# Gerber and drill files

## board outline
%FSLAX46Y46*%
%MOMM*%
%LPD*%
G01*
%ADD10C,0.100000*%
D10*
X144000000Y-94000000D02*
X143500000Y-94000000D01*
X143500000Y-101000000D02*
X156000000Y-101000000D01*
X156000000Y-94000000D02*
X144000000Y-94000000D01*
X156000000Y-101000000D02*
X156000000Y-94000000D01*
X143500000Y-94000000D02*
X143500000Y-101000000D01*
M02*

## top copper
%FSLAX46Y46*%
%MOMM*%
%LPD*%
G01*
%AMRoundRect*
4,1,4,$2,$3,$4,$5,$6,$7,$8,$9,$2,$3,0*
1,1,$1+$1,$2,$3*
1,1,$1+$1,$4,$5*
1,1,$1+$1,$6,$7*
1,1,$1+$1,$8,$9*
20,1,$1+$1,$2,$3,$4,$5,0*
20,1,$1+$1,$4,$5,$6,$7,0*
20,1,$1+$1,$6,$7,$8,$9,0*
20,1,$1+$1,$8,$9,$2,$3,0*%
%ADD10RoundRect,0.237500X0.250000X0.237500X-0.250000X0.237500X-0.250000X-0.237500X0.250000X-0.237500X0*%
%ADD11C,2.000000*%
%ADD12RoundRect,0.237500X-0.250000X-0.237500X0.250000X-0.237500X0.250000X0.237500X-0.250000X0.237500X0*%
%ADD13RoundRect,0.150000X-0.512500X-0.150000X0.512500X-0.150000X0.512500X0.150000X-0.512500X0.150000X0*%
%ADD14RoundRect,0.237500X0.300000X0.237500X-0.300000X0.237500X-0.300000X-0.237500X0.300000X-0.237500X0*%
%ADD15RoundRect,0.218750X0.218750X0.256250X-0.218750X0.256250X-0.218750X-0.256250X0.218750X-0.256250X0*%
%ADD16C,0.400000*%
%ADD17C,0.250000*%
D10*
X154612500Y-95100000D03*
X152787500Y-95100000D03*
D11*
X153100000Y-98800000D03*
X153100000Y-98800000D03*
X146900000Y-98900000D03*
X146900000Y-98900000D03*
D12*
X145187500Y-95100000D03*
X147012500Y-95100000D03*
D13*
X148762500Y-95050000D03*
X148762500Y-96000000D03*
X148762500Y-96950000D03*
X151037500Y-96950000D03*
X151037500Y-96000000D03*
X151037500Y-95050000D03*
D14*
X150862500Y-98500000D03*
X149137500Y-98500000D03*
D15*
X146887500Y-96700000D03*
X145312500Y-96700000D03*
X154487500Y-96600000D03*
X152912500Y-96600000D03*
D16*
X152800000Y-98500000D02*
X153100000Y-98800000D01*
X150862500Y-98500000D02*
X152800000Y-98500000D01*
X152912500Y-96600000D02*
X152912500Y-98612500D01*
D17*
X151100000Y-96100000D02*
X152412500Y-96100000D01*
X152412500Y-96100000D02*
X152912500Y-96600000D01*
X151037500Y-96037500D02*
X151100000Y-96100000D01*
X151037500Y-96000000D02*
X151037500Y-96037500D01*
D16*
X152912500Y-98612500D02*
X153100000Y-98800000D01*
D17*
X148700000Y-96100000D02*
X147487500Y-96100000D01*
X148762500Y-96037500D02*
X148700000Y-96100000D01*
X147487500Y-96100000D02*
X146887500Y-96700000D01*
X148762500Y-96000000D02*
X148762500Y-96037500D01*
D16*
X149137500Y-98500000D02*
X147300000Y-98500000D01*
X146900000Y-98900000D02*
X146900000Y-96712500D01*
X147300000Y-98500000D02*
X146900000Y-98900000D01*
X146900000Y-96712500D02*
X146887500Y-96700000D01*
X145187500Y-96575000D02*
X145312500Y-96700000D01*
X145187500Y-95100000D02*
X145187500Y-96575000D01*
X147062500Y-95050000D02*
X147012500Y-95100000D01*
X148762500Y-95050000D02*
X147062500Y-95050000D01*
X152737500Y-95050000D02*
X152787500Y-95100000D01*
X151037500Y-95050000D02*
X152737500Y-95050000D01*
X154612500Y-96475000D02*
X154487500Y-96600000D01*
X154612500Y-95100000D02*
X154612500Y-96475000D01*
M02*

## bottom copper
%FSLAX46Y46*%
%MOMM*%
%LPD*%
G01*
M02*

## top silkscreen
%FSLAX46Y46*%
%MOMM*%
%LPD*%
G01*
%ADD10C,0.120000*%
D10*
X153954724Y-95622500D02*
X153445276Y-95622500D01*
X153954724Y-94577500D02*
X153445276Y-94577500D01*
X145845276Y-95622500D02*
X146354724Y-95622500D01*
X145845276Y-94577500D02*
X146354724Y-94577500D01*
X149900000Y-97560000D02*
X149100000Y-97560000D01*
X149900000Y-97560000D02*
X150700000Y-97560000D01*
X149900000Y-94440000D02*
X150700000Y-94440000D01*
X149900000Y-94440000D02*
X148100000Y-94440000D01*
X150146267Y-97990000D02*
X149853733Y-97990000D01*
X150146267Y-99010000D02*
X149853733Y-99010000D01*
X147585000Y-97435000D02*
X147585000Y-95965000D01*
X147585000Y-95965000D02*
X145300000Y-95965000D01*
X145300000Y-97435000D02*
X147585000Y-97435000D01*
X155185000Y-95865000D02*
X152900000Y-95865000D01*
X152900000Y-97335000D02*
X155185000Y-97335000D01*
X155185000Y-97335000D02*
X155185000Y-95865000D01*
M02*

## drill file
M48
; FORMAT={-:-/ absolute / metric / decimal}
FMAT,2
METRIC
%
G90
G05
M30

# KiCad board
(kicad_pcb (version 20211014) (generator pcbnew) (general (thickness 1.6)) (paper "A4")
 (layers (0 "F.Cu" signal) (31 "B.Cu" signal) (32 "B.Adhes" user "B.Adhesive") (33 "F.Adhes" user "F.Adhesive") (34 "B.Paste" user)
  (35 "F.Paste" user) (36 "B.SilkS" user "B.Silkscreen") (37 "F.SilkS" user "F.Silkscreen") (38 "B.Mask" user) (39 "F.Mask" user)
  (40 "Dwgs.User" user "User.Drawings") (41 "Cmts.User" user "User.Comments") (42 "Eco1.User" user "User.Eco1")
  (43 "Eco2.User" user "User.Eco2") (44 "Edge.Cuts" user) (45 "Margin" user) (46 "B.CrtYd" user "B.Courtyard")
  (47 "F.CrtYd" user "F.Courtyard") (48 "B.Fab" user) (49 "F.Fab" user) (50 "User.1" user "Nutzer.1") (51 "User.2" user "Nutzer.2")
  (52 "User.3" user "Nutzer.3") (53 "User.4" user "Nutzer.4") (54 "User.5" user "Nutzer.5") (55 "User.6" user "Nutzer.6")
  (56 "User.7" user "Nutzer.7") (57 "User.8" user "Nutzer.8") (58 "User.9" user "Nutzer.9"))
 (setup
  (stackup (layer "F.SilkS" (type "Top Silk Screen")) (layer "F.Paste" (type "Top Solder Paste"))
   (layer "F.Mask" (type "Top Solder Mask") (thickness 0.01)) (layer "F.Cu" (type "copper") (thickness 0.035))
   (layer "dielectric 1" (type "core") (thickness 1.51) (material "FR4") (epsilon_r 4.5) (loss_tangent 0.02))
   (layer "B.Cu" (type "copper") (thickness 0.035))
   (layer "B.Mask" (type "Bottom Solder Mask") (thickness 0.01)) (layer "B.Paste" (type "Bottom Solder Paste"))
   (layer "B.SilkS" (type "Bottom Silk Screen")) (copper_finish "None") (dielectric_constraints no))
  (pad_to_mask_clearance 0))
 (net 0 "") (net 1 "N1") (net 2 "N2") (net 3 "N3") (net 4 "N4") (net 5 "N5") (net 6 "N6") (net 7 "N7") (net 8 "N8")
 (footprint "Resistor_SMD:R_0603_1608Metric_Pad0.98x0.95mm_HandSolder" (layer "F.Cu") (at 153.7 95.1 180)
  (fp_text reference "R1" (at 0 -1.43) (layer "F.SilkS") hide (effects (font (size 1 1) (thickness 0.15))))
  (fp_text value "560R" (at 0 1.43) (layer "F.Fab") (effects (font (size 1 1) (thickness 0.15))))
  (fp_line (start -0.254724 -0.5225) (end 0.254724 -0.5225) (layer "F.SilkS") (width 0.12))
  (fp_line (start -0.254724 0.5225) (end 0.254724 0.5225) (layer "F.SilkS") (width 0.12))
  (pad "1" smd roundrect (at -0.9125 0 180) (size 0.975 0.95) (layers "F.Cu" "F.Paste" "F.Mask") (roundrect_rratio 0.25) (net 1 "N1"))
  (pad "2" smd roundrect (at 0.9125 0 180) (size 0.975 0.95) (layers "F.Cu" "F.Paste" "F.Mask") (roundrect_rratio 0.25) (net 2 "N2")))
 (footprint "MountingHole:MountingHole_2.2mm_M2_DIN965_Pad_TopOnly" (layer "F.Cu") (at 153.1 98.8)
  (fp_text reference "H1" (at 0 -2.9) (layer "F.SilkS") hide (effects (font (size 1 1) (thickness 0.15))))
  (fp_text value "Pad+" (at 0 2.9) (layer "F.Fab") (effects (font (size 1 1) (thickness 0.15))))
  (pad "1" smd circle (at 0 0) (size 2 2) (layers "F.Cu" "F.Paste" "F.Mask") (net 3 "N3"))
  (pad "1" smd circle (at 0 0) (size 2 2) (layers "F.Cu" "F.Paste" "F.Mask") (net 3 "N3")))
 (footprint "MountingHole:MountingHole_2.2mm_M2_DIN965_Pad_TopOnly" (layer "F.Cu") (at 146.9 98.9)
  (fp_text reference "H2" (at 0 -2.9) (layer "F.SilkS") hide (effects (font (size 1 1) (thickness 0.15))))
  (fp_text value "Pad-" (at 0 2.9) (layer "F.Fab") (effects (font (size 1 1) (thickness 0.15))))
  (pad "1" smd circle (at 0 0) (size 2 2) (layers "F.Cu" "F.Paste" "F.Mask") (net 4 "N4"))
  (pad "1" smd circle (at 0 0) (size 2 2) (layers "F.Cu" "F.Paste" "F.Mask") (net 4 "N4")))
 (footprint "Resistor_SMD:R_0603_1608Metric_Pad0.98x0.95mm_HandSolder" (layer "F.Cu") (at 146.1 95.1)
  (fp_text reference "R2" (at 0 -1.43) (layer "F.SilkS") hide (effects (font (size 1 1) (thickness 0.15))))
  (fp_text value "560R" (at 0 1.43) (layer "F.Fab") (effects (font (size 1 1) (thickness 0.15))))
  (fp_line (start -0.254724 0.5225) (end 0.254724 0.5225) (layer "F.SilkS") (width 0.12))
  (fp_line (start -0.254724 -0.5225) (end 0.254724 -0.5225) (layer "F.SilkS") (width 0.12))
  (pad "1" smd roundrect (at -0.9125 0) (size 0.975 0.95) (layers "F.Cu" "F.Paste" "F.Mask") (roundrect_rratio 0.25) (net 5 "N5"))
  (pad "2" smd roundrect (at 0.9125 0) (size 0.975 0.95) (layers "F.Cu" "F.Paste" "F.Mask") (roundrect_rratio 0.25) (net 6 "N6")))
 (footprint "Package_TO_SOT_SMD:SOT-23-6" (layer "F.Cu") (at 149.9 96)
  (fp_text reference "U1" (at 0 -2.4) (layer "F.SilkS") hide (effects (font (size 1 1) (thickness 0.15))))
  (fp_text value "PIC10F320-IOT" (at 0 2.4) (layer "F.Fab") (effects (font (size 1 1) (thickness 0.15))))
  (fp_line (start 0 1.56) (end -0.8 1.56) (layer "F.SilkS") (width 0.12))
  (fp_line (start 0 1.56) (end 0.8 1.56) (layer "F.SilkS") (width 0.12))
  (fp_line (start 0 -1.56) (end 0.8 -1.56) (layer "F.SilkS") (width 0.12))
  (fp_line (start 0 -1.56) (end -1.8 -1.56) (layer "F.SilkS") (width 0.12))
  (pad "1" smd roundrect (at -1.1375 -0.95) (size 1.325 0.6) (layers "F.Cu" "F.Paste" "F.Mask") (roundrect_rratio 0.25) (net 6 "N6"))
  (pad "2" smd roundrect (at -1.1375 0) (size 1.325 0.6) (layers "F.Cu" "F.Paste" "F.Mask") (roundrect_rratio 0.25) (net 4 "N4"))
  (pad "3" smd roundrect (at -1.1375 0.95) (size 1.325 0.6) (layers "F.Cu" "F.Paste" "F.Mask") (roundrect_rratio 0.25) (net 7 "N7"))
  (pad "4" smd roundrect (at 1.1375 0.95) (size 1.325 0.6) (layers "F.Cu" "F.Paste" "F.Mask") (roundrect_rratio 0.25) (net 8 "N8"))
  (pad "5" smd roundrect (at 1.1375 0) (size 1.325 0.6) (layers "F.Cu" "F.Paste" "F.Mask") (roundrect_rratio 0.25) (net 3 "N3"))
  (pad "6" smd roundrect (at 1.1375 -0.95) (size 1.325 0.6) (layers "F.Cu" "F.Paste" "F.Mask") (roundrect_rratio 0.25) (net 2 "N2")))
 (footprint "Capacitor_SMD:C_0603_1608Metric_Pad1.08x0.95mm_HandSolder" (layer "F.Cu") (at 150 98.5 180)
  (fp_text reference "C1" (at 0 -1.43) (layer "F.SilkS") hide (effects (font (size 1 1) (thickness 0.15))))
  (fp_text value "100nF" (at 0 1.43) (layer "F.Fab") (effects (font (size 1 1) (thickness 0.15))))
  (fp_line (start -0.146267 0.51) (end 0.146267 0.51) (layer "F.SilkS") (width 0.12))
  (fp_line (start -0.146267 -0.51) (end 0.146267 -0.51) (layer "F.SilkS") (width 0.12))
  (pad "1" smd roundrect (at -0.8625 0 180) (size 1.075 0.95) (layers "F.Cu" "F.Paste" "F.Mask") (roundrect_rratio 0.25) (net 3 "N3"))
  (pad "2" smd roundrect (at 0.8625 0 180) (size 1.075 0.95) (layers "F.Cu" "F.Paste" "F.Mask") (roundrect_rratio 0.25) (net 4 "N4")))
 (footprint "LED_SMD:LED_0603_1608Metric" (layer "F.Cu") (at 146.1 96.7 180)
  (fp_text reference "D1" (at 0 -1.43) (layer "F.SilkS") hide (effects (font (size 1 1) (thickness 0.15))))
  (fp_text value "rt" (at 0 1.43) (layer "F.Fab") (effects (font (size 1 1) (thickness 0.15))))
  (fp_line (start -1.485 -0.735) (end -1.485 0.735) (layer "F.SilkS") (width 0.12))
  (fp_line (start -1.485 0.735) (end 0.8 0.735) (layer "F.SilkS") (width 0.12))
  (fp_line (start 0.8 -0.735) (end -1.485 -0.735) (layer "F.SilkS") (width 0.12))
  (pad "1" smd roundrect (at -0.7875 0 180) (size 0.875 0.95) (layers "F.Cu" "F.Paste" "F.Mask") (roundrect_rratio 0.25) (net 4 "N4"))
  (pad "2" smd roundrect (at 0.7875 0 180) (size 0.875 0.95) (layers "F.Cu" "F.Paste" "F.Mask") (roundrect_rratio 0.25) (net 5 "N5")))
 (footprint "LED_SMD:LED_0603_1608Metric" (layer "F.Cu") (at 153.7 96.6 180)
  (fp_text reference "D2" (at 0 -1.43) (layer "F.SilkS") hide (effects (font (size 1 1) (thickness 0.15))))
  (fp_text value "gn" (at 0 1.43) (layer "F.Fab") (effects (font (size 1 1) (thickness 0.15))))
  (fp_line (start -1.485 0.735) (end 0.8 0.735) (layer "F.SilkS") (width 0.12))
  (fp_line (start 0.8 -0.735) (end -1.485 -0.735) (layer "F.SilkS") (width 0.12))
  (fp_line (start -1.485 -0.735) (end -1.485 0.735) (layer "F.SilkS") (width 0.12))
  (pad "1" smd roundrect (at -0.7875 0 180) (size 0.875 0.95) (layers "F.Cu" "F.Paste" "F.Mask") (roundrect_rratio 0.25) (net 1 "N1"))
  (pad "2" smd roundrect (at 0.7875 0 180) (size 0.875 0.95) (layers "F.Cu" "F.Paste" "F.Mask") (roundrect_rratio 0.25) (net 3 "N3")))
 (gr_line (start 144 94) (end 143.5 94) (layer "Edge.Cuts") (width 0.1))
 (gr_line (start 143.5 101) (end 156 101) (layer "Edge.Cuts") (width 0.1))
 (gr_line (start 156 94) (end 144 94) (layer "Edge.Cuts") (width 0.1))
 (gr_line (start 156 101) (end 156 94) (layer "Edge.Cuts") (width 0.1))
 (gr_line (start 143.5 94) (end 143.5 101) (layer "Edge.Cuts") (width 0.1))
 (segment (start 152.8 98.5) (end 153.1 98.8) (width 0.4) (layer "F.Cu") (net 3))
 (segment (start 150.8625 98.5) (end 152.8 98.5) (width 0.4) (layer "F.Cu") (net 3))
 (segment (start 152.9125 96.6) (end 152.9125 98.6125) (width 0.4) (layer "F.Cu") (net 3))
 (segment (start 151.1 96.1) (end 152.4125 96.1) (width 0.25) (layer "F.Cu") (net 3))
 (segment (start 152.4125 96.1) (end 152.9125 96.6) (width 0.25) (layer "F.Cu") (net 3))
 (segment (start 151.0375 96.0375) (end 151.1 96.1) (width 0.25) (layer "F.Cu") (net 3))
 (segment (start 151.0375 96) (end 151.0375 96.0375) (width 0.25) (layer "F.Cu") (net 3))
 (segment (start 152.9125 98.6125) (end 153.1 98.8) (width 0.4) (layer "F.Cu") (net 3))
 (segment (start 148.7 96.1) (end 147.4875 96.1) (width 0.25) (layer "F.Cu") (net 4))
 (segment (start 148.7625 96.0375) (end 148.7 96.1) (width 0.25) (layer "F.Cu") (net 4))
 (segment (start 147.4875 96.1) (end 146.8875 96.7) (width 0.25) (layer "F.Cu") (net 4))
 (segment (start 148.7625 96) (end 148.7625 96.0375) (width 0.25) (layer "F.Cu") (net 4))
 (segment (start 149.1375 98.5) (end 147.3 98.5) (width 0.4) (layer "F.Cu") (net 4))
 (segment (start 146.9 98.9) (end 146.9 96.7125) (width 0.4) (layer "F.Cu") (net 4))
 (segment (start 147.3 98.5) (end 146.9 98.9) (width 0.4) (layer "F.Cu") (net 4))
 (segment (start 146.9 96.7125) (end 146.8875 96.7) (width 0.4) (layer "F.Cu") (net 4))
 (segment (start 145.1875 96.575) (end 145.3125 96.7) (width 0.4) (layer "F.Cu") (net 5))
 (segment (start 145.1875 95.1) (end 145.1875 96.575) (width 0.4) (layer "F.Cu") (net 5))
 (segment (start 147.0625 95.05) (end 147.0125 95.1) (width 0.4) (layer "F.Cu") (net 6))
 (segment (start 148.7625 95.05) (end 147.0625 95.05) (width 0.4) (layer "F.Cu") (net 6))
 (segment (start 152.7375 95.05) (end 152.7875 95.1) (width 0.4) (layer "F.Cu") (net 2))
 (segment (start 151.0375 95.05) (end 152.7375 95.05) (width 0.4) (layer "F.Cu") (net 2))
 (segment (start 154.6125 96.475) (end 154.4875 96.6) (width 0.4) (layer "F.Cu") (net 1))
 (segment (start 154.6125 95.1) (end 154.6125 96.475) (width 0.4) (layer "F.Cu") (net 1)))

